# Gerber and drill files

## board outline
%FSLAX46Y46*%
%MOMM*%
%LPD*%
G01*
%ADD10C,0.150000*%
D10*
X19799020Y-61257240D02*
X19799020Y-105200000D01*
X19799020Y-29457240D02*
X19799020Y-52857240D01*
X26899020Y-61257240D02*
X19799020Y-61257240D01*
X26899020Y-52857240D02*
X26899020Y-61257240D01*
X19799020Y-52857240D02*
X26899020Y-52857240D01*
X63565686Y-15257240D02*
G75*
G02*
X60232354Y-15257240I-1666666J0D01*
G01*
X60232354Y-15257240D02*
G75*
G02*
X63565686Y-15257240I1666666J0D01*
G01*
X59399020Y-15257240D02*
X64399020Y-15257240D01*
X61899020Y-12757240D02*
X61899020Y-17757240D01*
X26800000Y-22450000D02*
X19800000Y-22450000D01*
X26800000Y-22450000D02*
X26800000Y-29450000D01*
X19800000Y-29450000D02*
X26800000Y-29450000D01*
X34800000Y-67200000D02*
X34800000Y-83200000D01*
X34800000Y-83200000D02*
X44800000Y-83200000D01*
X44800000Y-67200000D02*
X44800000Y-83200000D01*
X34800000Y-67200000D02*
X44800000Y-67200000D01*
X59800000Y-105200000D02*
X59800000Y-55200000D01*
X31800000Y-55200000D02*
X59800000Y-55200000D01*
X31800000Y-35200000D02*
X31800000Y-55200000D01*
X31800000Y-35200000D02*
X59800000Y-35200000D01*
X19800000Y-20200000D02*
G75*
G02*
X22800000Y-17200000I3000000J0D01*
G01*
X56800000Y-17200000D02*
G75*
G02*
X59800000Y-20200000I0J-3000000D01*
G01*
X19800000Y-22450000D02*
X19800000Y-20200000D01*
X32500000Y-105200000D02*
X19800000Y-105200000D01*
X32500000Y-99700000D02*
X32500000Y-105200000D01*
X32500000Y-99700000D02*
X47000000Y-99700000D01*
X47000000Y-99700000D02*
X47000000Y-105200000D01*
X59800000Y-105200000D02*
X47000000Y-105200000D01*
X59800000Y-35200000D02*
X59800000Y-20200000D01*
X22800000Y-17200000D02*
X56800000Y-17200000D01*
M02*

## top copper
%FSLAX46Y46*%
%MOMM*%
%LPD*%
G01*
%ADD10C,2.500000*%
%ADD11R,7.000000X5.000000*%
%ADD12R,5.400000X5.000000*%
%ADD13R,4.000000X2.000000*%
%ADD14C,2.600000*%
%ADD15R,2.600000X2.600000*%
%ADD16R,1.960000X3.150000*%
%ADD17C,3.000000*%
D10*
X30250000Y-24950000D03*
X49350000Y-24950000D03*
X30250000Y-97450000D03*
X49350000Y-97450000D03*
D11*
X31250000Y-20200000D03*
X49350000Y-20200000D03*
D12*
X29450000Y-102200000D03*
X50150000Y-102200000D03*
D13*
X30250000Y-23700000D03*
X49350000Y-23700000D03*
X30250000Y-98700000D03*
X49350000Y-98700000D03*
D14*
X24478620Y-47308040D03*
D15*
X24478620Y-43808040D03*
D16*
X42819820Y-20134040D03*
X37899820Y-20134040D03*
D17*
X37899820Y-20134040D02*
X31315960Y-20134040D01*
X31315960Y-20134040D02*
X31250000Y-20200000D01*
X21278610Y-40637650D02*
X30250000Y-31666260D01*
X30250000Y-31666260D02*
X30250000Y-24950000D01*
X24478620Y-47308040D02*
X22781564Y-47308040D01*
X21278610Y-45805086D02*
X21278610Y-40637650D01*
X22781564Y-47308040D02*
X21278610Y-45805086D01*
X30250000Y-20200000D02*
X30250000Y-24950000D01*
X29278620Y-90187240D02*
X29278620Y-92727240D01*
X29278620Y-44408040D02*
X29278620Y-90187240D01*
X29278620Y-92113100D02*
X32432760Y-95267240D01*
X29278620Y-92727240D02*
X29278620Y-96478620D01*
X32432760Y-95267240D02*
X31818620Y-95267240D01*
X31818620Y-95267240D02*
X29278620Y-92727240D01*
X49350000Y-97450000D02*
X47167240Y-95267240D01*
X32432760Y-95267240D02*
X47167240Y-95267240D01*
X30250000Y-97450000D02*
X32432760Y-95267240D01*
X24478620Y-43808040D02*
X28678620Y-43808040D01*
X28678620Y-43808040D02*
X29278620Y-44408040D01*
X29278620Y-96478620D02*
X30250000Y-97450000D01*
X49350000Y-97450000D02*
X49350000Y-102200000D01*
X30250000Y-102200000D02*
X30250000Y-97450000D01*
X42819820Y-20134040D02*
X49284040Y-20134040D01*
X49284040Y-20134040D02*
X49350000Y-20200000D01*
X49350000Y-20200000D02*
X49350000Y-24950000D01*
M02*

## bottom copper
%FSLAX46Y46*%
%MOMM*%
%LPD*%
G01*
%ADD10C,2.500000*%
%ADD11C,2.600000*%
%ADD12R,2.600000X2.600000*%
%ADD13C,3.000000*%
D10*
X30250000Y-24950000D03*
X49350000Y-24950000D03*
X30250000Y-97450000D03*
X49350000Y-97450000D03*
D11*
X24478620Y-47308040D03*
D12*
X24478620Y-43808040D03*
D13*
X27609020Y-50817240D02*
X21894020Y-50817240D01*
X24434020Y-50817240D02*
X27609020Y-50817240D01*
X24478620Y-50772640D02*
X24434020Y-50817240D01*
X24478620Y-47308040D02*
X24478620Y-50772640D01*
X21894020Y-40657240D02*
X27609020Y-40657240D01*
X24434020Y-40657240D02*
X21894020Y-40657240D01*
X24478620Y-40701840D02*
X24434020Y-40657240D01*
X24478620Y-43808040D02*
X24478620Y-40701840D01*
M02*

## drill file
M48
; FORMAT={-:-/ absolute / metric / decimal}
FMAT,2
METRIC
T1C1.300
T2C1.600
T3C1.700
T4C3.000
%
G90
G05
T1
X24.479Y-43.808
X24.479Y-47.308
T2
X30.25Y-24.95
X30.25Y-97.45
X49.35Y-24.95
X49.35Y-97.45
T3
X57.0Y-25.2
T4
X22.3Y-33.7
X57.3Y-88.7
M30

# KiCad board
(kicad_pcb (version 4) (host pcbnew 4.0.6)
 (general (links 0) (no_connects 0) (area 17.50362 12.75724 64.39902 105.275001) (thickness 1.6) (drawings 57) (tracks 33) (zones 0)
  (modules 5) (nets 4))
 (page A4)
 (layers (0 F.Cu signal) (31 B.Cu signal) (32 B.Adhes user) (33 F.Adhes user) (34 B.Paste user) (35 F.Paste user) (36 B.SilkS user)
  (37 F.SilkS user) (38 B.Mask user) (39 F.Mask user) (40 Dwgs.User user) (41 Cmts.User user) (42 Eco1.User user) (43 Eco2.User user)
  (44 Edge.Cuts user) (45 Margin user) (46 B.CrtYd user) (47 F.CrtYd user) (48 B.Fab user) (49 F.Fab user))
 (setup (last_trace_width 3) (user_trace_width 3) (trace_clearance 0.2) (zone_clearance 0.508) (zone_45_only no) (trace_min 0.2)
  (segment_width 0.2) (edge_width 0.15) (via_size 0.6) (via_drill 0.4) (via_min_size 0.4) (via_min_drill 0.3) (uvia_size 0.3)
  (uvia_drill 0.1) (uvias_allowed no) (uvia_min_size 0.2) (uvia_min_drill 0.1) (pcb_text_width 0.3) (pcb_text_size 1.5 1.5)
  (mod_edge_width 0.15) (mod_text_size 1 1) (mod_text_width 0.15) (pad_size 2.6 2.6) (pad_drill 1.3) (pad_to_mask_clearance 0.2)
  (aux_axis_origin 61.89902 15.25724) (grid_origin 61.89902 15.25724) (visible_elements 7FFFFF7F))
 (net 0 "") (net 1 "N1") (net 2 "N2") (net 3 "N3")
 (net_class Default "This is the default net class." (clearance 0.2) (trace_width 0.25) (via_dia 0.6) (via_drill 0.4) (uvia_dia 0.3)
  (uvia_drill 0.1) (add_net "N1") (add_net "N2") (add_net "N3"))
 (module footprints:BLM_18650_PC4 (layer F.Cu) (at 39.8 61.2)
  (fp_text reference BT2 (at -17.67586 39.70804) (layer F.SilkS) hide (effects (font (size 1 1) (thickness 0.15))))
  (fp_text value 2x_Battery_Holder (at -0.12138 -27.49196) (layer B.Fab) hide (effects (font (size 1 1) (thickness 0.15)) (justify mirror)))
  (pad 1 thru_hole circle (at -9.55 -36.25) (size 2.5 2.5) (drill 1.6) (layers *.Cu *.Mask) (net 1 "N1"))
  (pad 2 thru_hole circle (at 9.55 -36.25) (size 2.5 2.5) (drill 1.6) (layers *.Cu *.Mask) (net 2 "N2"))
  (pad 3 thru_hole circle (at -9.55 36.25) (size 2.5 2.5) (drill 1.6) (layers *.Cu *.Mask) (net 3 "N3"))
  (pad 4 thru_hole circle (at 9.55 36.25) (size 2.5 2.5) (drill 1.6) (layers *.Cu *.Mask) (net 3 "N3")))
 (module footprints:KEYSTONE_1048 (layer F.Cu) (at 39.8 61.2)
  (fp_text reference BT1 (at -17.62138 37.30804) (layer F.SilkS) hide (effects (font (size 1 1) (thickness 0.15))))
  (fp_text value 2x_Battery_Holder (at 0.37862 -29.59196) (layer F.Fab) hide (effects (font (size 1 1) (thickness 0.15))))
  (pad 1 smd rect (at -8.55 -41) (size 7 5) (layers F.Cu F.Paste F.Mask) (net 1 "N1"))
  (pad 2 smd rect (at 9.55 -41) (size 7 5) (layers F.Cu F.Paste F.Mask) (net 2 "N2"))
  (pad 3 smd rect (at -10.35 41) (size 5.4 5) (layers F.Cu F.Paste F.Mask) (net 3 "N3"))
  (pad 4 smd rect (at 10.35 41) (size 5.4 5) (layers F.Cu F.Paste F.Mask) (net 3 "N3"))
  (pad "" np_thru_hole circle (at 17.2 -36) (size 1.7 1.7) (drill 1.7) (layers *.Cu *.Mask))
  (pad "" np_thru_hole circle (at -17.5 -27.5) (size 3 3) (drill 3) (layers *.Cu *.Mask))
  (pad "" np_thru_hole circle (at 17.5 27.5) (size 3 3) (drill 3) (layers *.Cu *.Mask))
  (pad 1 smd rect (at -9.55 -37.5) (size 4 2) (layers F.Cu F.Paste F.Mask) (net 1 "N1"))
  (pad 2 smd rect (at 9.55 -37.5) (size 4 2) (layers F.Cu F.Paste F.Mask) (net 2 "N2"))
  (pad 3 smd rect (at -9.55 37.5) (size 4 2) (layers F.Cu F.Paste F.Mask) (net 3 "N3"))
  (pad 4 smd rect (at 9.55 37.5) (size 4 2) (layers F.Cu F.Paste F.Mask) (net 3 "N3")))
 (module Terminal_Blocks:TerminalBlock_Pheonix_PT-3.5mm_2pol (layer F.Cu) (at 24.47862 43.80804 270)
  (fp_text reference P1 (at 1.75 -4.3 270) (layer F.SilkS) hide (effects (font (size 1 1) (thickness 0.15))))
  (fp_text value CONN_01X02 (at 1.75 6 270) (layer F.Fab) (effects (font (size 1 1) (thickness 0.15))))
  (pad 2 thru_hole circle (at 3.5 0 270) (size 2.6 2.6) (drill 1.3) (layers *.Cu *.Mask) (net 1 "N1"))
  (pad 1 thru_hole rect (at 0 0 270) (size 2.6 2.6) (drill 1.3) (layers *.Cu *.Mask) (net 3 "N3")))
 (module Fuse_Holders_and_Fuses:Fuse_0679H (layer F.Cu) (at 40.35982 20.13404)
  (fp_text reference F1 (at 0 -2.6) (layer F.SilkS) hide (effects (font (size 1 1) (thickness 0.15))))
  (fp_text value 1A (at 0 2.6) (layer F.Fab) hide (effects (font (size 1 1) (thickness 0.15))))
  (pad 2 smd rect (at 2.46 0) (size 1.96 3.15) (layers F.Cu F.Paste F.Mask) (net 2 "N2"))
  (pad 1 smd rect (at -2.46 0) (size 1.96 3.15) (layers F.Cu F.Paste F.Mask) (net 1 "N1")))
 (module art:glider (layer F.Cu) (at 29.69902 32.35724)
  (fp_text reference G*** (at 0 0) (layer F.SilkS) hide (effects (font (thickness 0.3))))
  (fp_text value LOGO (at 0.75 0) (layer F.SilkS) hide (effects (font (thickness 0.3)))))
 (gr_line (start 19.79902 61.25724) (end 19.79902 105.2) (layer Edge.Cuts) (width 0.15))
 (gr_line (start 19.79902 29.45724) (end 19.79902 52.85724) (layer Edge.Cuts) (width 0.15))
 (gr_line (start 26.89902 61.25724) (end 19.79902 61.25724) (layer Edge.Cuts) (width 0.15))
 (gr_line (start 26.89902 52.85724) (end 26.89902 61.25724) (layer Edge.Cuts) (width 0.15))
 (gr_line (start 19.79902 52.85724) (end 26.89902 52.85724) (layer Edge.Cuts) (width 0.15))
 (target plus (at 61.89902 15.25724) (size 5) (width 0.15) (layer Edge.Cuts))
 (gr_line (start 26.8 22.45) (end 19.8 22.45) (layer Edge.Cuts) (width 0.15))
 (gr_line (start 26.8 22.45) (end 26.8 29.45) (layer Edge.Cuts) (width 0.15))
 (gr_line (start 19.8 29.45) (end 26.8 29.45) (layer Edge.Cuts) (width 0.15))
 (gr_line (start 34.8 67.2) (end 34.8 83.2) (layer Edge.Cuts) (width 0.15))
 (gr_line (start 34.8 83.2) (end 44.8 83.2) (layer Edge.Cuts) (width 0.15))
 (gr_line (start 44.8 67.2) (end 44.8 83.2) (layer Edge.Cuts) (width 0.15))
 (gr_line (start 34.8 67.2) (end 44.8 67.2) (layer Edge.Cuts) (width 0.15))
 (gr_line (start 59.8 105.2) (end 59.8 55.2) (layer Edge.Cuts) (width 0.15))
 (gr_line (start 31.8 55.2) (end 59.8 55.2) (layer Edge.Cuts) (width 0.15))
 (gr_line (start 31.8 35.2) (end 31.8 55.2) (layer Edge.Cuts) (width 0.15))
 (gr_line (start 31.8 35.2) (end 59.8 35.2) (layer Edge.Cuts) (width 0.15))
 (gr_arc (start 22.8 20.2) (end 19.8 20.2) (angle 90) (layer Edge.Cuts) (width 0.15))
 (gr_arc (start 56.8 20.2) (end 56.8 17.2) (angle 90) (layer Edge.Cuts) (width 0.15))
 (gr_line (start 19.8 22.45) (end 19.8 20.2) (layer Edge.Cuts) (width 0.15))
 (gr_line (start 32.5 105.2) (end 19.8 105.2) (layer Edge.Cuts) (width 0.15))
 (gr_line (start 32.5 99.7) (end 32.5 105.2) (layer Edge.Cuts) (width 0.15))
 (gr_line (start 32.5 99.7) (end 47 99.7) (layer Edge.Cuts) (width 0.15))
 (gr_line (start 47 99.7) (end 47 105.2) (layer Edge.Cuts) (width 0.15))
 (gr_line (start 59.8 105.2) (end 47 105.2) (layer Edge.Cuts) (width 0.15))
 (gr_line (start 59.8 35.2) (end 59.8 20.2) (layer Edge.Cuts) (width 0.15))
 (gr_line (start 22.8 17.2) (end 56.8 17.2) (layer Edge.Cuts) (width 0.15))
 (segment (start 27.60902 50.81724) (end 21.89402 50.81724) (width 3) (layer B.Cu) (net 1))
 (segment (start 24.43402 50.81724) (end 27.60902 50.81724) (width 3) (layer B.Cu) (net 1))
 (segment (start 24.47862 50.77264) (end 24.43402 50.81724) (width 3) (layer B.Cu) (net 1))
 (segment (start 24.47862 47.30804) (end 24.47862 50.77264) (width 3) (layer B.Cu) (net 1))
 (segment (start 37.89982 20.13404) (end 31.31596 20.13404) (width 3) (layer F.Cu) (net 1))
 (segment (start 31.31596 20.13404) (end 31.25 20.2) (width 3) (layer F.Cu) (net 1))
 (segment (start 21.27861 40.63765) (end 30.25 31.66626) (width 3) (layer F.Cu) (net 1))
 (segment (start 30.25 31.66626) (end 30.25 24.95) (width 3) (layer F.Cu) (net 1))
 (segment (start 24.47862 47.30804) (end 22.781564 47.30804) (width 3) (layer F.Cu) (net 1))
 (segment (start 21.27861 45.805086) (end 21.27861 40.63765) (width 3) (layer F.Cu) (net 1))
 (segment (start 22.781564 47.30804) (end 21.27861 45.805086) (width 3) (layer F.Cu) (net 1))
 (segment (start 30.25 20.2) (end 30.25 24.95) (width 3) (layer F.Cu) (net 1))
 (segment (start 29.27862 90.18724) (end 29.27862 92.72724) (width 3) (layer F.Cu) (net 3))
 (segment (start 29.27862 44.40804) (end 29.27862 90.18724) (width 3) (layer F.Cu) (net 3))
 (segment (start 29.27862 92.1131) (end 32.43276 95.26724) (width 3) (layer F.Cu) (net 3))
 (segment (start 29.27862 92.72724) (end 29.27862 96.47862) (width 3) (layer F.Cu) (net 3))
 (segment (start 32.43276 95.26724) (end 31.81862 95.26724) (width 3) (layer F.Cu) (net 3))
 (segment (start 31.81862 95.26724) (end 29.27862 92.72724) (width 3) (layer F.Cu) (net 3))
 (segment (start 49.35 97.45) (end 47.16724 95.26724) (width 3) (layer F.Cu) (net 3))
 (segment (start 32.43276 95.26724) (end 47.16724 95.26724) (width 3) (layer F.Cu) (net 3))
 (segment (start 30.25 97.45) (end 32.43276 95.26724) (width 3) (layer F.Cu) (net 3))
 (segment (start 21.89402 40.65724) (end 27.60902 40.65724) (width 3) (layer B.Cu) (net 3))
 (segment (start 24.43402 40.65724) (end 21.89402 40.65724) (width 3) (layer B.Cu) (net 3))
 (segment (start 24.47862 40.70184) (end 24.43402 40.65724) (width 3) (layer B.Cu) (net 3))
 (segment (start 24.47862 43.80804) (end 24.47862 40.70184) (width 3) (layer B.Cu) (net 3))
 (segment (start 24.47862 43.80804) (end 28.67862 43.80804) (width 3) (layer F.Cu) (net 3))
 (segment (start 28.67862 43.80804) (end 29.27862 44.40804) (width 3) (layer F.Cu) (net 3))
 (segment (start 29.27862 96.47862) (end 30.25 97.45) (width 3) (layer F.Cu) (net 3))
 (segment (start 49.35 97.45) (end 49.35 102.2) (width 3) (layer F.Cu) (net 3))
 (segment (start 30.25 102.2) (end 30.25 97.45) (width 3) (layer F.Cu) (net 3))
 (segment (start 42.81982 20.13404) (end 49.28404 20.13404) (width 3) (layer F.Cu) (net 2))
 (segment (start 49.28404 20.13404) (end 49.35 20.2) (width 3) (layer F.Cu) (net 2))
 (segment (start 49.35 20.2) (end 49.35 24.95) (width 3) (layer F.Cu) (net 2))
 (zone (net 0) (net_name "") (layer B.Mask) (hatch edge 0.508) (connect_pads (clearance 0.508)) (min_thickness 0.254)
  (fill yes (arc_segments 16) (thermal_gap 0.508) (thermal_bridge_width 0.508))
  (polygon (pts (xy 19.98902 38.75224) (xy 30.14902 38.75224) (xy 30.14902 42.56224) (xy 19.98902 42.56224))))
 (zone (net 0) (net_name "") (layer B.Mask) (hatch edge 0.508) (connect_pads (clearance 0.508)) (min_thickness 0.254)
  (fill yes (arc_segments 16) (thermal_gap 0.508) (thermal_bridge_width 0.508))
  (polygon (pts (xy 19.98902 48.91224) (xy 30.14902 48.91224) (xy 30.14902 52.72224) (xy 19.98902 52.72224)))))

